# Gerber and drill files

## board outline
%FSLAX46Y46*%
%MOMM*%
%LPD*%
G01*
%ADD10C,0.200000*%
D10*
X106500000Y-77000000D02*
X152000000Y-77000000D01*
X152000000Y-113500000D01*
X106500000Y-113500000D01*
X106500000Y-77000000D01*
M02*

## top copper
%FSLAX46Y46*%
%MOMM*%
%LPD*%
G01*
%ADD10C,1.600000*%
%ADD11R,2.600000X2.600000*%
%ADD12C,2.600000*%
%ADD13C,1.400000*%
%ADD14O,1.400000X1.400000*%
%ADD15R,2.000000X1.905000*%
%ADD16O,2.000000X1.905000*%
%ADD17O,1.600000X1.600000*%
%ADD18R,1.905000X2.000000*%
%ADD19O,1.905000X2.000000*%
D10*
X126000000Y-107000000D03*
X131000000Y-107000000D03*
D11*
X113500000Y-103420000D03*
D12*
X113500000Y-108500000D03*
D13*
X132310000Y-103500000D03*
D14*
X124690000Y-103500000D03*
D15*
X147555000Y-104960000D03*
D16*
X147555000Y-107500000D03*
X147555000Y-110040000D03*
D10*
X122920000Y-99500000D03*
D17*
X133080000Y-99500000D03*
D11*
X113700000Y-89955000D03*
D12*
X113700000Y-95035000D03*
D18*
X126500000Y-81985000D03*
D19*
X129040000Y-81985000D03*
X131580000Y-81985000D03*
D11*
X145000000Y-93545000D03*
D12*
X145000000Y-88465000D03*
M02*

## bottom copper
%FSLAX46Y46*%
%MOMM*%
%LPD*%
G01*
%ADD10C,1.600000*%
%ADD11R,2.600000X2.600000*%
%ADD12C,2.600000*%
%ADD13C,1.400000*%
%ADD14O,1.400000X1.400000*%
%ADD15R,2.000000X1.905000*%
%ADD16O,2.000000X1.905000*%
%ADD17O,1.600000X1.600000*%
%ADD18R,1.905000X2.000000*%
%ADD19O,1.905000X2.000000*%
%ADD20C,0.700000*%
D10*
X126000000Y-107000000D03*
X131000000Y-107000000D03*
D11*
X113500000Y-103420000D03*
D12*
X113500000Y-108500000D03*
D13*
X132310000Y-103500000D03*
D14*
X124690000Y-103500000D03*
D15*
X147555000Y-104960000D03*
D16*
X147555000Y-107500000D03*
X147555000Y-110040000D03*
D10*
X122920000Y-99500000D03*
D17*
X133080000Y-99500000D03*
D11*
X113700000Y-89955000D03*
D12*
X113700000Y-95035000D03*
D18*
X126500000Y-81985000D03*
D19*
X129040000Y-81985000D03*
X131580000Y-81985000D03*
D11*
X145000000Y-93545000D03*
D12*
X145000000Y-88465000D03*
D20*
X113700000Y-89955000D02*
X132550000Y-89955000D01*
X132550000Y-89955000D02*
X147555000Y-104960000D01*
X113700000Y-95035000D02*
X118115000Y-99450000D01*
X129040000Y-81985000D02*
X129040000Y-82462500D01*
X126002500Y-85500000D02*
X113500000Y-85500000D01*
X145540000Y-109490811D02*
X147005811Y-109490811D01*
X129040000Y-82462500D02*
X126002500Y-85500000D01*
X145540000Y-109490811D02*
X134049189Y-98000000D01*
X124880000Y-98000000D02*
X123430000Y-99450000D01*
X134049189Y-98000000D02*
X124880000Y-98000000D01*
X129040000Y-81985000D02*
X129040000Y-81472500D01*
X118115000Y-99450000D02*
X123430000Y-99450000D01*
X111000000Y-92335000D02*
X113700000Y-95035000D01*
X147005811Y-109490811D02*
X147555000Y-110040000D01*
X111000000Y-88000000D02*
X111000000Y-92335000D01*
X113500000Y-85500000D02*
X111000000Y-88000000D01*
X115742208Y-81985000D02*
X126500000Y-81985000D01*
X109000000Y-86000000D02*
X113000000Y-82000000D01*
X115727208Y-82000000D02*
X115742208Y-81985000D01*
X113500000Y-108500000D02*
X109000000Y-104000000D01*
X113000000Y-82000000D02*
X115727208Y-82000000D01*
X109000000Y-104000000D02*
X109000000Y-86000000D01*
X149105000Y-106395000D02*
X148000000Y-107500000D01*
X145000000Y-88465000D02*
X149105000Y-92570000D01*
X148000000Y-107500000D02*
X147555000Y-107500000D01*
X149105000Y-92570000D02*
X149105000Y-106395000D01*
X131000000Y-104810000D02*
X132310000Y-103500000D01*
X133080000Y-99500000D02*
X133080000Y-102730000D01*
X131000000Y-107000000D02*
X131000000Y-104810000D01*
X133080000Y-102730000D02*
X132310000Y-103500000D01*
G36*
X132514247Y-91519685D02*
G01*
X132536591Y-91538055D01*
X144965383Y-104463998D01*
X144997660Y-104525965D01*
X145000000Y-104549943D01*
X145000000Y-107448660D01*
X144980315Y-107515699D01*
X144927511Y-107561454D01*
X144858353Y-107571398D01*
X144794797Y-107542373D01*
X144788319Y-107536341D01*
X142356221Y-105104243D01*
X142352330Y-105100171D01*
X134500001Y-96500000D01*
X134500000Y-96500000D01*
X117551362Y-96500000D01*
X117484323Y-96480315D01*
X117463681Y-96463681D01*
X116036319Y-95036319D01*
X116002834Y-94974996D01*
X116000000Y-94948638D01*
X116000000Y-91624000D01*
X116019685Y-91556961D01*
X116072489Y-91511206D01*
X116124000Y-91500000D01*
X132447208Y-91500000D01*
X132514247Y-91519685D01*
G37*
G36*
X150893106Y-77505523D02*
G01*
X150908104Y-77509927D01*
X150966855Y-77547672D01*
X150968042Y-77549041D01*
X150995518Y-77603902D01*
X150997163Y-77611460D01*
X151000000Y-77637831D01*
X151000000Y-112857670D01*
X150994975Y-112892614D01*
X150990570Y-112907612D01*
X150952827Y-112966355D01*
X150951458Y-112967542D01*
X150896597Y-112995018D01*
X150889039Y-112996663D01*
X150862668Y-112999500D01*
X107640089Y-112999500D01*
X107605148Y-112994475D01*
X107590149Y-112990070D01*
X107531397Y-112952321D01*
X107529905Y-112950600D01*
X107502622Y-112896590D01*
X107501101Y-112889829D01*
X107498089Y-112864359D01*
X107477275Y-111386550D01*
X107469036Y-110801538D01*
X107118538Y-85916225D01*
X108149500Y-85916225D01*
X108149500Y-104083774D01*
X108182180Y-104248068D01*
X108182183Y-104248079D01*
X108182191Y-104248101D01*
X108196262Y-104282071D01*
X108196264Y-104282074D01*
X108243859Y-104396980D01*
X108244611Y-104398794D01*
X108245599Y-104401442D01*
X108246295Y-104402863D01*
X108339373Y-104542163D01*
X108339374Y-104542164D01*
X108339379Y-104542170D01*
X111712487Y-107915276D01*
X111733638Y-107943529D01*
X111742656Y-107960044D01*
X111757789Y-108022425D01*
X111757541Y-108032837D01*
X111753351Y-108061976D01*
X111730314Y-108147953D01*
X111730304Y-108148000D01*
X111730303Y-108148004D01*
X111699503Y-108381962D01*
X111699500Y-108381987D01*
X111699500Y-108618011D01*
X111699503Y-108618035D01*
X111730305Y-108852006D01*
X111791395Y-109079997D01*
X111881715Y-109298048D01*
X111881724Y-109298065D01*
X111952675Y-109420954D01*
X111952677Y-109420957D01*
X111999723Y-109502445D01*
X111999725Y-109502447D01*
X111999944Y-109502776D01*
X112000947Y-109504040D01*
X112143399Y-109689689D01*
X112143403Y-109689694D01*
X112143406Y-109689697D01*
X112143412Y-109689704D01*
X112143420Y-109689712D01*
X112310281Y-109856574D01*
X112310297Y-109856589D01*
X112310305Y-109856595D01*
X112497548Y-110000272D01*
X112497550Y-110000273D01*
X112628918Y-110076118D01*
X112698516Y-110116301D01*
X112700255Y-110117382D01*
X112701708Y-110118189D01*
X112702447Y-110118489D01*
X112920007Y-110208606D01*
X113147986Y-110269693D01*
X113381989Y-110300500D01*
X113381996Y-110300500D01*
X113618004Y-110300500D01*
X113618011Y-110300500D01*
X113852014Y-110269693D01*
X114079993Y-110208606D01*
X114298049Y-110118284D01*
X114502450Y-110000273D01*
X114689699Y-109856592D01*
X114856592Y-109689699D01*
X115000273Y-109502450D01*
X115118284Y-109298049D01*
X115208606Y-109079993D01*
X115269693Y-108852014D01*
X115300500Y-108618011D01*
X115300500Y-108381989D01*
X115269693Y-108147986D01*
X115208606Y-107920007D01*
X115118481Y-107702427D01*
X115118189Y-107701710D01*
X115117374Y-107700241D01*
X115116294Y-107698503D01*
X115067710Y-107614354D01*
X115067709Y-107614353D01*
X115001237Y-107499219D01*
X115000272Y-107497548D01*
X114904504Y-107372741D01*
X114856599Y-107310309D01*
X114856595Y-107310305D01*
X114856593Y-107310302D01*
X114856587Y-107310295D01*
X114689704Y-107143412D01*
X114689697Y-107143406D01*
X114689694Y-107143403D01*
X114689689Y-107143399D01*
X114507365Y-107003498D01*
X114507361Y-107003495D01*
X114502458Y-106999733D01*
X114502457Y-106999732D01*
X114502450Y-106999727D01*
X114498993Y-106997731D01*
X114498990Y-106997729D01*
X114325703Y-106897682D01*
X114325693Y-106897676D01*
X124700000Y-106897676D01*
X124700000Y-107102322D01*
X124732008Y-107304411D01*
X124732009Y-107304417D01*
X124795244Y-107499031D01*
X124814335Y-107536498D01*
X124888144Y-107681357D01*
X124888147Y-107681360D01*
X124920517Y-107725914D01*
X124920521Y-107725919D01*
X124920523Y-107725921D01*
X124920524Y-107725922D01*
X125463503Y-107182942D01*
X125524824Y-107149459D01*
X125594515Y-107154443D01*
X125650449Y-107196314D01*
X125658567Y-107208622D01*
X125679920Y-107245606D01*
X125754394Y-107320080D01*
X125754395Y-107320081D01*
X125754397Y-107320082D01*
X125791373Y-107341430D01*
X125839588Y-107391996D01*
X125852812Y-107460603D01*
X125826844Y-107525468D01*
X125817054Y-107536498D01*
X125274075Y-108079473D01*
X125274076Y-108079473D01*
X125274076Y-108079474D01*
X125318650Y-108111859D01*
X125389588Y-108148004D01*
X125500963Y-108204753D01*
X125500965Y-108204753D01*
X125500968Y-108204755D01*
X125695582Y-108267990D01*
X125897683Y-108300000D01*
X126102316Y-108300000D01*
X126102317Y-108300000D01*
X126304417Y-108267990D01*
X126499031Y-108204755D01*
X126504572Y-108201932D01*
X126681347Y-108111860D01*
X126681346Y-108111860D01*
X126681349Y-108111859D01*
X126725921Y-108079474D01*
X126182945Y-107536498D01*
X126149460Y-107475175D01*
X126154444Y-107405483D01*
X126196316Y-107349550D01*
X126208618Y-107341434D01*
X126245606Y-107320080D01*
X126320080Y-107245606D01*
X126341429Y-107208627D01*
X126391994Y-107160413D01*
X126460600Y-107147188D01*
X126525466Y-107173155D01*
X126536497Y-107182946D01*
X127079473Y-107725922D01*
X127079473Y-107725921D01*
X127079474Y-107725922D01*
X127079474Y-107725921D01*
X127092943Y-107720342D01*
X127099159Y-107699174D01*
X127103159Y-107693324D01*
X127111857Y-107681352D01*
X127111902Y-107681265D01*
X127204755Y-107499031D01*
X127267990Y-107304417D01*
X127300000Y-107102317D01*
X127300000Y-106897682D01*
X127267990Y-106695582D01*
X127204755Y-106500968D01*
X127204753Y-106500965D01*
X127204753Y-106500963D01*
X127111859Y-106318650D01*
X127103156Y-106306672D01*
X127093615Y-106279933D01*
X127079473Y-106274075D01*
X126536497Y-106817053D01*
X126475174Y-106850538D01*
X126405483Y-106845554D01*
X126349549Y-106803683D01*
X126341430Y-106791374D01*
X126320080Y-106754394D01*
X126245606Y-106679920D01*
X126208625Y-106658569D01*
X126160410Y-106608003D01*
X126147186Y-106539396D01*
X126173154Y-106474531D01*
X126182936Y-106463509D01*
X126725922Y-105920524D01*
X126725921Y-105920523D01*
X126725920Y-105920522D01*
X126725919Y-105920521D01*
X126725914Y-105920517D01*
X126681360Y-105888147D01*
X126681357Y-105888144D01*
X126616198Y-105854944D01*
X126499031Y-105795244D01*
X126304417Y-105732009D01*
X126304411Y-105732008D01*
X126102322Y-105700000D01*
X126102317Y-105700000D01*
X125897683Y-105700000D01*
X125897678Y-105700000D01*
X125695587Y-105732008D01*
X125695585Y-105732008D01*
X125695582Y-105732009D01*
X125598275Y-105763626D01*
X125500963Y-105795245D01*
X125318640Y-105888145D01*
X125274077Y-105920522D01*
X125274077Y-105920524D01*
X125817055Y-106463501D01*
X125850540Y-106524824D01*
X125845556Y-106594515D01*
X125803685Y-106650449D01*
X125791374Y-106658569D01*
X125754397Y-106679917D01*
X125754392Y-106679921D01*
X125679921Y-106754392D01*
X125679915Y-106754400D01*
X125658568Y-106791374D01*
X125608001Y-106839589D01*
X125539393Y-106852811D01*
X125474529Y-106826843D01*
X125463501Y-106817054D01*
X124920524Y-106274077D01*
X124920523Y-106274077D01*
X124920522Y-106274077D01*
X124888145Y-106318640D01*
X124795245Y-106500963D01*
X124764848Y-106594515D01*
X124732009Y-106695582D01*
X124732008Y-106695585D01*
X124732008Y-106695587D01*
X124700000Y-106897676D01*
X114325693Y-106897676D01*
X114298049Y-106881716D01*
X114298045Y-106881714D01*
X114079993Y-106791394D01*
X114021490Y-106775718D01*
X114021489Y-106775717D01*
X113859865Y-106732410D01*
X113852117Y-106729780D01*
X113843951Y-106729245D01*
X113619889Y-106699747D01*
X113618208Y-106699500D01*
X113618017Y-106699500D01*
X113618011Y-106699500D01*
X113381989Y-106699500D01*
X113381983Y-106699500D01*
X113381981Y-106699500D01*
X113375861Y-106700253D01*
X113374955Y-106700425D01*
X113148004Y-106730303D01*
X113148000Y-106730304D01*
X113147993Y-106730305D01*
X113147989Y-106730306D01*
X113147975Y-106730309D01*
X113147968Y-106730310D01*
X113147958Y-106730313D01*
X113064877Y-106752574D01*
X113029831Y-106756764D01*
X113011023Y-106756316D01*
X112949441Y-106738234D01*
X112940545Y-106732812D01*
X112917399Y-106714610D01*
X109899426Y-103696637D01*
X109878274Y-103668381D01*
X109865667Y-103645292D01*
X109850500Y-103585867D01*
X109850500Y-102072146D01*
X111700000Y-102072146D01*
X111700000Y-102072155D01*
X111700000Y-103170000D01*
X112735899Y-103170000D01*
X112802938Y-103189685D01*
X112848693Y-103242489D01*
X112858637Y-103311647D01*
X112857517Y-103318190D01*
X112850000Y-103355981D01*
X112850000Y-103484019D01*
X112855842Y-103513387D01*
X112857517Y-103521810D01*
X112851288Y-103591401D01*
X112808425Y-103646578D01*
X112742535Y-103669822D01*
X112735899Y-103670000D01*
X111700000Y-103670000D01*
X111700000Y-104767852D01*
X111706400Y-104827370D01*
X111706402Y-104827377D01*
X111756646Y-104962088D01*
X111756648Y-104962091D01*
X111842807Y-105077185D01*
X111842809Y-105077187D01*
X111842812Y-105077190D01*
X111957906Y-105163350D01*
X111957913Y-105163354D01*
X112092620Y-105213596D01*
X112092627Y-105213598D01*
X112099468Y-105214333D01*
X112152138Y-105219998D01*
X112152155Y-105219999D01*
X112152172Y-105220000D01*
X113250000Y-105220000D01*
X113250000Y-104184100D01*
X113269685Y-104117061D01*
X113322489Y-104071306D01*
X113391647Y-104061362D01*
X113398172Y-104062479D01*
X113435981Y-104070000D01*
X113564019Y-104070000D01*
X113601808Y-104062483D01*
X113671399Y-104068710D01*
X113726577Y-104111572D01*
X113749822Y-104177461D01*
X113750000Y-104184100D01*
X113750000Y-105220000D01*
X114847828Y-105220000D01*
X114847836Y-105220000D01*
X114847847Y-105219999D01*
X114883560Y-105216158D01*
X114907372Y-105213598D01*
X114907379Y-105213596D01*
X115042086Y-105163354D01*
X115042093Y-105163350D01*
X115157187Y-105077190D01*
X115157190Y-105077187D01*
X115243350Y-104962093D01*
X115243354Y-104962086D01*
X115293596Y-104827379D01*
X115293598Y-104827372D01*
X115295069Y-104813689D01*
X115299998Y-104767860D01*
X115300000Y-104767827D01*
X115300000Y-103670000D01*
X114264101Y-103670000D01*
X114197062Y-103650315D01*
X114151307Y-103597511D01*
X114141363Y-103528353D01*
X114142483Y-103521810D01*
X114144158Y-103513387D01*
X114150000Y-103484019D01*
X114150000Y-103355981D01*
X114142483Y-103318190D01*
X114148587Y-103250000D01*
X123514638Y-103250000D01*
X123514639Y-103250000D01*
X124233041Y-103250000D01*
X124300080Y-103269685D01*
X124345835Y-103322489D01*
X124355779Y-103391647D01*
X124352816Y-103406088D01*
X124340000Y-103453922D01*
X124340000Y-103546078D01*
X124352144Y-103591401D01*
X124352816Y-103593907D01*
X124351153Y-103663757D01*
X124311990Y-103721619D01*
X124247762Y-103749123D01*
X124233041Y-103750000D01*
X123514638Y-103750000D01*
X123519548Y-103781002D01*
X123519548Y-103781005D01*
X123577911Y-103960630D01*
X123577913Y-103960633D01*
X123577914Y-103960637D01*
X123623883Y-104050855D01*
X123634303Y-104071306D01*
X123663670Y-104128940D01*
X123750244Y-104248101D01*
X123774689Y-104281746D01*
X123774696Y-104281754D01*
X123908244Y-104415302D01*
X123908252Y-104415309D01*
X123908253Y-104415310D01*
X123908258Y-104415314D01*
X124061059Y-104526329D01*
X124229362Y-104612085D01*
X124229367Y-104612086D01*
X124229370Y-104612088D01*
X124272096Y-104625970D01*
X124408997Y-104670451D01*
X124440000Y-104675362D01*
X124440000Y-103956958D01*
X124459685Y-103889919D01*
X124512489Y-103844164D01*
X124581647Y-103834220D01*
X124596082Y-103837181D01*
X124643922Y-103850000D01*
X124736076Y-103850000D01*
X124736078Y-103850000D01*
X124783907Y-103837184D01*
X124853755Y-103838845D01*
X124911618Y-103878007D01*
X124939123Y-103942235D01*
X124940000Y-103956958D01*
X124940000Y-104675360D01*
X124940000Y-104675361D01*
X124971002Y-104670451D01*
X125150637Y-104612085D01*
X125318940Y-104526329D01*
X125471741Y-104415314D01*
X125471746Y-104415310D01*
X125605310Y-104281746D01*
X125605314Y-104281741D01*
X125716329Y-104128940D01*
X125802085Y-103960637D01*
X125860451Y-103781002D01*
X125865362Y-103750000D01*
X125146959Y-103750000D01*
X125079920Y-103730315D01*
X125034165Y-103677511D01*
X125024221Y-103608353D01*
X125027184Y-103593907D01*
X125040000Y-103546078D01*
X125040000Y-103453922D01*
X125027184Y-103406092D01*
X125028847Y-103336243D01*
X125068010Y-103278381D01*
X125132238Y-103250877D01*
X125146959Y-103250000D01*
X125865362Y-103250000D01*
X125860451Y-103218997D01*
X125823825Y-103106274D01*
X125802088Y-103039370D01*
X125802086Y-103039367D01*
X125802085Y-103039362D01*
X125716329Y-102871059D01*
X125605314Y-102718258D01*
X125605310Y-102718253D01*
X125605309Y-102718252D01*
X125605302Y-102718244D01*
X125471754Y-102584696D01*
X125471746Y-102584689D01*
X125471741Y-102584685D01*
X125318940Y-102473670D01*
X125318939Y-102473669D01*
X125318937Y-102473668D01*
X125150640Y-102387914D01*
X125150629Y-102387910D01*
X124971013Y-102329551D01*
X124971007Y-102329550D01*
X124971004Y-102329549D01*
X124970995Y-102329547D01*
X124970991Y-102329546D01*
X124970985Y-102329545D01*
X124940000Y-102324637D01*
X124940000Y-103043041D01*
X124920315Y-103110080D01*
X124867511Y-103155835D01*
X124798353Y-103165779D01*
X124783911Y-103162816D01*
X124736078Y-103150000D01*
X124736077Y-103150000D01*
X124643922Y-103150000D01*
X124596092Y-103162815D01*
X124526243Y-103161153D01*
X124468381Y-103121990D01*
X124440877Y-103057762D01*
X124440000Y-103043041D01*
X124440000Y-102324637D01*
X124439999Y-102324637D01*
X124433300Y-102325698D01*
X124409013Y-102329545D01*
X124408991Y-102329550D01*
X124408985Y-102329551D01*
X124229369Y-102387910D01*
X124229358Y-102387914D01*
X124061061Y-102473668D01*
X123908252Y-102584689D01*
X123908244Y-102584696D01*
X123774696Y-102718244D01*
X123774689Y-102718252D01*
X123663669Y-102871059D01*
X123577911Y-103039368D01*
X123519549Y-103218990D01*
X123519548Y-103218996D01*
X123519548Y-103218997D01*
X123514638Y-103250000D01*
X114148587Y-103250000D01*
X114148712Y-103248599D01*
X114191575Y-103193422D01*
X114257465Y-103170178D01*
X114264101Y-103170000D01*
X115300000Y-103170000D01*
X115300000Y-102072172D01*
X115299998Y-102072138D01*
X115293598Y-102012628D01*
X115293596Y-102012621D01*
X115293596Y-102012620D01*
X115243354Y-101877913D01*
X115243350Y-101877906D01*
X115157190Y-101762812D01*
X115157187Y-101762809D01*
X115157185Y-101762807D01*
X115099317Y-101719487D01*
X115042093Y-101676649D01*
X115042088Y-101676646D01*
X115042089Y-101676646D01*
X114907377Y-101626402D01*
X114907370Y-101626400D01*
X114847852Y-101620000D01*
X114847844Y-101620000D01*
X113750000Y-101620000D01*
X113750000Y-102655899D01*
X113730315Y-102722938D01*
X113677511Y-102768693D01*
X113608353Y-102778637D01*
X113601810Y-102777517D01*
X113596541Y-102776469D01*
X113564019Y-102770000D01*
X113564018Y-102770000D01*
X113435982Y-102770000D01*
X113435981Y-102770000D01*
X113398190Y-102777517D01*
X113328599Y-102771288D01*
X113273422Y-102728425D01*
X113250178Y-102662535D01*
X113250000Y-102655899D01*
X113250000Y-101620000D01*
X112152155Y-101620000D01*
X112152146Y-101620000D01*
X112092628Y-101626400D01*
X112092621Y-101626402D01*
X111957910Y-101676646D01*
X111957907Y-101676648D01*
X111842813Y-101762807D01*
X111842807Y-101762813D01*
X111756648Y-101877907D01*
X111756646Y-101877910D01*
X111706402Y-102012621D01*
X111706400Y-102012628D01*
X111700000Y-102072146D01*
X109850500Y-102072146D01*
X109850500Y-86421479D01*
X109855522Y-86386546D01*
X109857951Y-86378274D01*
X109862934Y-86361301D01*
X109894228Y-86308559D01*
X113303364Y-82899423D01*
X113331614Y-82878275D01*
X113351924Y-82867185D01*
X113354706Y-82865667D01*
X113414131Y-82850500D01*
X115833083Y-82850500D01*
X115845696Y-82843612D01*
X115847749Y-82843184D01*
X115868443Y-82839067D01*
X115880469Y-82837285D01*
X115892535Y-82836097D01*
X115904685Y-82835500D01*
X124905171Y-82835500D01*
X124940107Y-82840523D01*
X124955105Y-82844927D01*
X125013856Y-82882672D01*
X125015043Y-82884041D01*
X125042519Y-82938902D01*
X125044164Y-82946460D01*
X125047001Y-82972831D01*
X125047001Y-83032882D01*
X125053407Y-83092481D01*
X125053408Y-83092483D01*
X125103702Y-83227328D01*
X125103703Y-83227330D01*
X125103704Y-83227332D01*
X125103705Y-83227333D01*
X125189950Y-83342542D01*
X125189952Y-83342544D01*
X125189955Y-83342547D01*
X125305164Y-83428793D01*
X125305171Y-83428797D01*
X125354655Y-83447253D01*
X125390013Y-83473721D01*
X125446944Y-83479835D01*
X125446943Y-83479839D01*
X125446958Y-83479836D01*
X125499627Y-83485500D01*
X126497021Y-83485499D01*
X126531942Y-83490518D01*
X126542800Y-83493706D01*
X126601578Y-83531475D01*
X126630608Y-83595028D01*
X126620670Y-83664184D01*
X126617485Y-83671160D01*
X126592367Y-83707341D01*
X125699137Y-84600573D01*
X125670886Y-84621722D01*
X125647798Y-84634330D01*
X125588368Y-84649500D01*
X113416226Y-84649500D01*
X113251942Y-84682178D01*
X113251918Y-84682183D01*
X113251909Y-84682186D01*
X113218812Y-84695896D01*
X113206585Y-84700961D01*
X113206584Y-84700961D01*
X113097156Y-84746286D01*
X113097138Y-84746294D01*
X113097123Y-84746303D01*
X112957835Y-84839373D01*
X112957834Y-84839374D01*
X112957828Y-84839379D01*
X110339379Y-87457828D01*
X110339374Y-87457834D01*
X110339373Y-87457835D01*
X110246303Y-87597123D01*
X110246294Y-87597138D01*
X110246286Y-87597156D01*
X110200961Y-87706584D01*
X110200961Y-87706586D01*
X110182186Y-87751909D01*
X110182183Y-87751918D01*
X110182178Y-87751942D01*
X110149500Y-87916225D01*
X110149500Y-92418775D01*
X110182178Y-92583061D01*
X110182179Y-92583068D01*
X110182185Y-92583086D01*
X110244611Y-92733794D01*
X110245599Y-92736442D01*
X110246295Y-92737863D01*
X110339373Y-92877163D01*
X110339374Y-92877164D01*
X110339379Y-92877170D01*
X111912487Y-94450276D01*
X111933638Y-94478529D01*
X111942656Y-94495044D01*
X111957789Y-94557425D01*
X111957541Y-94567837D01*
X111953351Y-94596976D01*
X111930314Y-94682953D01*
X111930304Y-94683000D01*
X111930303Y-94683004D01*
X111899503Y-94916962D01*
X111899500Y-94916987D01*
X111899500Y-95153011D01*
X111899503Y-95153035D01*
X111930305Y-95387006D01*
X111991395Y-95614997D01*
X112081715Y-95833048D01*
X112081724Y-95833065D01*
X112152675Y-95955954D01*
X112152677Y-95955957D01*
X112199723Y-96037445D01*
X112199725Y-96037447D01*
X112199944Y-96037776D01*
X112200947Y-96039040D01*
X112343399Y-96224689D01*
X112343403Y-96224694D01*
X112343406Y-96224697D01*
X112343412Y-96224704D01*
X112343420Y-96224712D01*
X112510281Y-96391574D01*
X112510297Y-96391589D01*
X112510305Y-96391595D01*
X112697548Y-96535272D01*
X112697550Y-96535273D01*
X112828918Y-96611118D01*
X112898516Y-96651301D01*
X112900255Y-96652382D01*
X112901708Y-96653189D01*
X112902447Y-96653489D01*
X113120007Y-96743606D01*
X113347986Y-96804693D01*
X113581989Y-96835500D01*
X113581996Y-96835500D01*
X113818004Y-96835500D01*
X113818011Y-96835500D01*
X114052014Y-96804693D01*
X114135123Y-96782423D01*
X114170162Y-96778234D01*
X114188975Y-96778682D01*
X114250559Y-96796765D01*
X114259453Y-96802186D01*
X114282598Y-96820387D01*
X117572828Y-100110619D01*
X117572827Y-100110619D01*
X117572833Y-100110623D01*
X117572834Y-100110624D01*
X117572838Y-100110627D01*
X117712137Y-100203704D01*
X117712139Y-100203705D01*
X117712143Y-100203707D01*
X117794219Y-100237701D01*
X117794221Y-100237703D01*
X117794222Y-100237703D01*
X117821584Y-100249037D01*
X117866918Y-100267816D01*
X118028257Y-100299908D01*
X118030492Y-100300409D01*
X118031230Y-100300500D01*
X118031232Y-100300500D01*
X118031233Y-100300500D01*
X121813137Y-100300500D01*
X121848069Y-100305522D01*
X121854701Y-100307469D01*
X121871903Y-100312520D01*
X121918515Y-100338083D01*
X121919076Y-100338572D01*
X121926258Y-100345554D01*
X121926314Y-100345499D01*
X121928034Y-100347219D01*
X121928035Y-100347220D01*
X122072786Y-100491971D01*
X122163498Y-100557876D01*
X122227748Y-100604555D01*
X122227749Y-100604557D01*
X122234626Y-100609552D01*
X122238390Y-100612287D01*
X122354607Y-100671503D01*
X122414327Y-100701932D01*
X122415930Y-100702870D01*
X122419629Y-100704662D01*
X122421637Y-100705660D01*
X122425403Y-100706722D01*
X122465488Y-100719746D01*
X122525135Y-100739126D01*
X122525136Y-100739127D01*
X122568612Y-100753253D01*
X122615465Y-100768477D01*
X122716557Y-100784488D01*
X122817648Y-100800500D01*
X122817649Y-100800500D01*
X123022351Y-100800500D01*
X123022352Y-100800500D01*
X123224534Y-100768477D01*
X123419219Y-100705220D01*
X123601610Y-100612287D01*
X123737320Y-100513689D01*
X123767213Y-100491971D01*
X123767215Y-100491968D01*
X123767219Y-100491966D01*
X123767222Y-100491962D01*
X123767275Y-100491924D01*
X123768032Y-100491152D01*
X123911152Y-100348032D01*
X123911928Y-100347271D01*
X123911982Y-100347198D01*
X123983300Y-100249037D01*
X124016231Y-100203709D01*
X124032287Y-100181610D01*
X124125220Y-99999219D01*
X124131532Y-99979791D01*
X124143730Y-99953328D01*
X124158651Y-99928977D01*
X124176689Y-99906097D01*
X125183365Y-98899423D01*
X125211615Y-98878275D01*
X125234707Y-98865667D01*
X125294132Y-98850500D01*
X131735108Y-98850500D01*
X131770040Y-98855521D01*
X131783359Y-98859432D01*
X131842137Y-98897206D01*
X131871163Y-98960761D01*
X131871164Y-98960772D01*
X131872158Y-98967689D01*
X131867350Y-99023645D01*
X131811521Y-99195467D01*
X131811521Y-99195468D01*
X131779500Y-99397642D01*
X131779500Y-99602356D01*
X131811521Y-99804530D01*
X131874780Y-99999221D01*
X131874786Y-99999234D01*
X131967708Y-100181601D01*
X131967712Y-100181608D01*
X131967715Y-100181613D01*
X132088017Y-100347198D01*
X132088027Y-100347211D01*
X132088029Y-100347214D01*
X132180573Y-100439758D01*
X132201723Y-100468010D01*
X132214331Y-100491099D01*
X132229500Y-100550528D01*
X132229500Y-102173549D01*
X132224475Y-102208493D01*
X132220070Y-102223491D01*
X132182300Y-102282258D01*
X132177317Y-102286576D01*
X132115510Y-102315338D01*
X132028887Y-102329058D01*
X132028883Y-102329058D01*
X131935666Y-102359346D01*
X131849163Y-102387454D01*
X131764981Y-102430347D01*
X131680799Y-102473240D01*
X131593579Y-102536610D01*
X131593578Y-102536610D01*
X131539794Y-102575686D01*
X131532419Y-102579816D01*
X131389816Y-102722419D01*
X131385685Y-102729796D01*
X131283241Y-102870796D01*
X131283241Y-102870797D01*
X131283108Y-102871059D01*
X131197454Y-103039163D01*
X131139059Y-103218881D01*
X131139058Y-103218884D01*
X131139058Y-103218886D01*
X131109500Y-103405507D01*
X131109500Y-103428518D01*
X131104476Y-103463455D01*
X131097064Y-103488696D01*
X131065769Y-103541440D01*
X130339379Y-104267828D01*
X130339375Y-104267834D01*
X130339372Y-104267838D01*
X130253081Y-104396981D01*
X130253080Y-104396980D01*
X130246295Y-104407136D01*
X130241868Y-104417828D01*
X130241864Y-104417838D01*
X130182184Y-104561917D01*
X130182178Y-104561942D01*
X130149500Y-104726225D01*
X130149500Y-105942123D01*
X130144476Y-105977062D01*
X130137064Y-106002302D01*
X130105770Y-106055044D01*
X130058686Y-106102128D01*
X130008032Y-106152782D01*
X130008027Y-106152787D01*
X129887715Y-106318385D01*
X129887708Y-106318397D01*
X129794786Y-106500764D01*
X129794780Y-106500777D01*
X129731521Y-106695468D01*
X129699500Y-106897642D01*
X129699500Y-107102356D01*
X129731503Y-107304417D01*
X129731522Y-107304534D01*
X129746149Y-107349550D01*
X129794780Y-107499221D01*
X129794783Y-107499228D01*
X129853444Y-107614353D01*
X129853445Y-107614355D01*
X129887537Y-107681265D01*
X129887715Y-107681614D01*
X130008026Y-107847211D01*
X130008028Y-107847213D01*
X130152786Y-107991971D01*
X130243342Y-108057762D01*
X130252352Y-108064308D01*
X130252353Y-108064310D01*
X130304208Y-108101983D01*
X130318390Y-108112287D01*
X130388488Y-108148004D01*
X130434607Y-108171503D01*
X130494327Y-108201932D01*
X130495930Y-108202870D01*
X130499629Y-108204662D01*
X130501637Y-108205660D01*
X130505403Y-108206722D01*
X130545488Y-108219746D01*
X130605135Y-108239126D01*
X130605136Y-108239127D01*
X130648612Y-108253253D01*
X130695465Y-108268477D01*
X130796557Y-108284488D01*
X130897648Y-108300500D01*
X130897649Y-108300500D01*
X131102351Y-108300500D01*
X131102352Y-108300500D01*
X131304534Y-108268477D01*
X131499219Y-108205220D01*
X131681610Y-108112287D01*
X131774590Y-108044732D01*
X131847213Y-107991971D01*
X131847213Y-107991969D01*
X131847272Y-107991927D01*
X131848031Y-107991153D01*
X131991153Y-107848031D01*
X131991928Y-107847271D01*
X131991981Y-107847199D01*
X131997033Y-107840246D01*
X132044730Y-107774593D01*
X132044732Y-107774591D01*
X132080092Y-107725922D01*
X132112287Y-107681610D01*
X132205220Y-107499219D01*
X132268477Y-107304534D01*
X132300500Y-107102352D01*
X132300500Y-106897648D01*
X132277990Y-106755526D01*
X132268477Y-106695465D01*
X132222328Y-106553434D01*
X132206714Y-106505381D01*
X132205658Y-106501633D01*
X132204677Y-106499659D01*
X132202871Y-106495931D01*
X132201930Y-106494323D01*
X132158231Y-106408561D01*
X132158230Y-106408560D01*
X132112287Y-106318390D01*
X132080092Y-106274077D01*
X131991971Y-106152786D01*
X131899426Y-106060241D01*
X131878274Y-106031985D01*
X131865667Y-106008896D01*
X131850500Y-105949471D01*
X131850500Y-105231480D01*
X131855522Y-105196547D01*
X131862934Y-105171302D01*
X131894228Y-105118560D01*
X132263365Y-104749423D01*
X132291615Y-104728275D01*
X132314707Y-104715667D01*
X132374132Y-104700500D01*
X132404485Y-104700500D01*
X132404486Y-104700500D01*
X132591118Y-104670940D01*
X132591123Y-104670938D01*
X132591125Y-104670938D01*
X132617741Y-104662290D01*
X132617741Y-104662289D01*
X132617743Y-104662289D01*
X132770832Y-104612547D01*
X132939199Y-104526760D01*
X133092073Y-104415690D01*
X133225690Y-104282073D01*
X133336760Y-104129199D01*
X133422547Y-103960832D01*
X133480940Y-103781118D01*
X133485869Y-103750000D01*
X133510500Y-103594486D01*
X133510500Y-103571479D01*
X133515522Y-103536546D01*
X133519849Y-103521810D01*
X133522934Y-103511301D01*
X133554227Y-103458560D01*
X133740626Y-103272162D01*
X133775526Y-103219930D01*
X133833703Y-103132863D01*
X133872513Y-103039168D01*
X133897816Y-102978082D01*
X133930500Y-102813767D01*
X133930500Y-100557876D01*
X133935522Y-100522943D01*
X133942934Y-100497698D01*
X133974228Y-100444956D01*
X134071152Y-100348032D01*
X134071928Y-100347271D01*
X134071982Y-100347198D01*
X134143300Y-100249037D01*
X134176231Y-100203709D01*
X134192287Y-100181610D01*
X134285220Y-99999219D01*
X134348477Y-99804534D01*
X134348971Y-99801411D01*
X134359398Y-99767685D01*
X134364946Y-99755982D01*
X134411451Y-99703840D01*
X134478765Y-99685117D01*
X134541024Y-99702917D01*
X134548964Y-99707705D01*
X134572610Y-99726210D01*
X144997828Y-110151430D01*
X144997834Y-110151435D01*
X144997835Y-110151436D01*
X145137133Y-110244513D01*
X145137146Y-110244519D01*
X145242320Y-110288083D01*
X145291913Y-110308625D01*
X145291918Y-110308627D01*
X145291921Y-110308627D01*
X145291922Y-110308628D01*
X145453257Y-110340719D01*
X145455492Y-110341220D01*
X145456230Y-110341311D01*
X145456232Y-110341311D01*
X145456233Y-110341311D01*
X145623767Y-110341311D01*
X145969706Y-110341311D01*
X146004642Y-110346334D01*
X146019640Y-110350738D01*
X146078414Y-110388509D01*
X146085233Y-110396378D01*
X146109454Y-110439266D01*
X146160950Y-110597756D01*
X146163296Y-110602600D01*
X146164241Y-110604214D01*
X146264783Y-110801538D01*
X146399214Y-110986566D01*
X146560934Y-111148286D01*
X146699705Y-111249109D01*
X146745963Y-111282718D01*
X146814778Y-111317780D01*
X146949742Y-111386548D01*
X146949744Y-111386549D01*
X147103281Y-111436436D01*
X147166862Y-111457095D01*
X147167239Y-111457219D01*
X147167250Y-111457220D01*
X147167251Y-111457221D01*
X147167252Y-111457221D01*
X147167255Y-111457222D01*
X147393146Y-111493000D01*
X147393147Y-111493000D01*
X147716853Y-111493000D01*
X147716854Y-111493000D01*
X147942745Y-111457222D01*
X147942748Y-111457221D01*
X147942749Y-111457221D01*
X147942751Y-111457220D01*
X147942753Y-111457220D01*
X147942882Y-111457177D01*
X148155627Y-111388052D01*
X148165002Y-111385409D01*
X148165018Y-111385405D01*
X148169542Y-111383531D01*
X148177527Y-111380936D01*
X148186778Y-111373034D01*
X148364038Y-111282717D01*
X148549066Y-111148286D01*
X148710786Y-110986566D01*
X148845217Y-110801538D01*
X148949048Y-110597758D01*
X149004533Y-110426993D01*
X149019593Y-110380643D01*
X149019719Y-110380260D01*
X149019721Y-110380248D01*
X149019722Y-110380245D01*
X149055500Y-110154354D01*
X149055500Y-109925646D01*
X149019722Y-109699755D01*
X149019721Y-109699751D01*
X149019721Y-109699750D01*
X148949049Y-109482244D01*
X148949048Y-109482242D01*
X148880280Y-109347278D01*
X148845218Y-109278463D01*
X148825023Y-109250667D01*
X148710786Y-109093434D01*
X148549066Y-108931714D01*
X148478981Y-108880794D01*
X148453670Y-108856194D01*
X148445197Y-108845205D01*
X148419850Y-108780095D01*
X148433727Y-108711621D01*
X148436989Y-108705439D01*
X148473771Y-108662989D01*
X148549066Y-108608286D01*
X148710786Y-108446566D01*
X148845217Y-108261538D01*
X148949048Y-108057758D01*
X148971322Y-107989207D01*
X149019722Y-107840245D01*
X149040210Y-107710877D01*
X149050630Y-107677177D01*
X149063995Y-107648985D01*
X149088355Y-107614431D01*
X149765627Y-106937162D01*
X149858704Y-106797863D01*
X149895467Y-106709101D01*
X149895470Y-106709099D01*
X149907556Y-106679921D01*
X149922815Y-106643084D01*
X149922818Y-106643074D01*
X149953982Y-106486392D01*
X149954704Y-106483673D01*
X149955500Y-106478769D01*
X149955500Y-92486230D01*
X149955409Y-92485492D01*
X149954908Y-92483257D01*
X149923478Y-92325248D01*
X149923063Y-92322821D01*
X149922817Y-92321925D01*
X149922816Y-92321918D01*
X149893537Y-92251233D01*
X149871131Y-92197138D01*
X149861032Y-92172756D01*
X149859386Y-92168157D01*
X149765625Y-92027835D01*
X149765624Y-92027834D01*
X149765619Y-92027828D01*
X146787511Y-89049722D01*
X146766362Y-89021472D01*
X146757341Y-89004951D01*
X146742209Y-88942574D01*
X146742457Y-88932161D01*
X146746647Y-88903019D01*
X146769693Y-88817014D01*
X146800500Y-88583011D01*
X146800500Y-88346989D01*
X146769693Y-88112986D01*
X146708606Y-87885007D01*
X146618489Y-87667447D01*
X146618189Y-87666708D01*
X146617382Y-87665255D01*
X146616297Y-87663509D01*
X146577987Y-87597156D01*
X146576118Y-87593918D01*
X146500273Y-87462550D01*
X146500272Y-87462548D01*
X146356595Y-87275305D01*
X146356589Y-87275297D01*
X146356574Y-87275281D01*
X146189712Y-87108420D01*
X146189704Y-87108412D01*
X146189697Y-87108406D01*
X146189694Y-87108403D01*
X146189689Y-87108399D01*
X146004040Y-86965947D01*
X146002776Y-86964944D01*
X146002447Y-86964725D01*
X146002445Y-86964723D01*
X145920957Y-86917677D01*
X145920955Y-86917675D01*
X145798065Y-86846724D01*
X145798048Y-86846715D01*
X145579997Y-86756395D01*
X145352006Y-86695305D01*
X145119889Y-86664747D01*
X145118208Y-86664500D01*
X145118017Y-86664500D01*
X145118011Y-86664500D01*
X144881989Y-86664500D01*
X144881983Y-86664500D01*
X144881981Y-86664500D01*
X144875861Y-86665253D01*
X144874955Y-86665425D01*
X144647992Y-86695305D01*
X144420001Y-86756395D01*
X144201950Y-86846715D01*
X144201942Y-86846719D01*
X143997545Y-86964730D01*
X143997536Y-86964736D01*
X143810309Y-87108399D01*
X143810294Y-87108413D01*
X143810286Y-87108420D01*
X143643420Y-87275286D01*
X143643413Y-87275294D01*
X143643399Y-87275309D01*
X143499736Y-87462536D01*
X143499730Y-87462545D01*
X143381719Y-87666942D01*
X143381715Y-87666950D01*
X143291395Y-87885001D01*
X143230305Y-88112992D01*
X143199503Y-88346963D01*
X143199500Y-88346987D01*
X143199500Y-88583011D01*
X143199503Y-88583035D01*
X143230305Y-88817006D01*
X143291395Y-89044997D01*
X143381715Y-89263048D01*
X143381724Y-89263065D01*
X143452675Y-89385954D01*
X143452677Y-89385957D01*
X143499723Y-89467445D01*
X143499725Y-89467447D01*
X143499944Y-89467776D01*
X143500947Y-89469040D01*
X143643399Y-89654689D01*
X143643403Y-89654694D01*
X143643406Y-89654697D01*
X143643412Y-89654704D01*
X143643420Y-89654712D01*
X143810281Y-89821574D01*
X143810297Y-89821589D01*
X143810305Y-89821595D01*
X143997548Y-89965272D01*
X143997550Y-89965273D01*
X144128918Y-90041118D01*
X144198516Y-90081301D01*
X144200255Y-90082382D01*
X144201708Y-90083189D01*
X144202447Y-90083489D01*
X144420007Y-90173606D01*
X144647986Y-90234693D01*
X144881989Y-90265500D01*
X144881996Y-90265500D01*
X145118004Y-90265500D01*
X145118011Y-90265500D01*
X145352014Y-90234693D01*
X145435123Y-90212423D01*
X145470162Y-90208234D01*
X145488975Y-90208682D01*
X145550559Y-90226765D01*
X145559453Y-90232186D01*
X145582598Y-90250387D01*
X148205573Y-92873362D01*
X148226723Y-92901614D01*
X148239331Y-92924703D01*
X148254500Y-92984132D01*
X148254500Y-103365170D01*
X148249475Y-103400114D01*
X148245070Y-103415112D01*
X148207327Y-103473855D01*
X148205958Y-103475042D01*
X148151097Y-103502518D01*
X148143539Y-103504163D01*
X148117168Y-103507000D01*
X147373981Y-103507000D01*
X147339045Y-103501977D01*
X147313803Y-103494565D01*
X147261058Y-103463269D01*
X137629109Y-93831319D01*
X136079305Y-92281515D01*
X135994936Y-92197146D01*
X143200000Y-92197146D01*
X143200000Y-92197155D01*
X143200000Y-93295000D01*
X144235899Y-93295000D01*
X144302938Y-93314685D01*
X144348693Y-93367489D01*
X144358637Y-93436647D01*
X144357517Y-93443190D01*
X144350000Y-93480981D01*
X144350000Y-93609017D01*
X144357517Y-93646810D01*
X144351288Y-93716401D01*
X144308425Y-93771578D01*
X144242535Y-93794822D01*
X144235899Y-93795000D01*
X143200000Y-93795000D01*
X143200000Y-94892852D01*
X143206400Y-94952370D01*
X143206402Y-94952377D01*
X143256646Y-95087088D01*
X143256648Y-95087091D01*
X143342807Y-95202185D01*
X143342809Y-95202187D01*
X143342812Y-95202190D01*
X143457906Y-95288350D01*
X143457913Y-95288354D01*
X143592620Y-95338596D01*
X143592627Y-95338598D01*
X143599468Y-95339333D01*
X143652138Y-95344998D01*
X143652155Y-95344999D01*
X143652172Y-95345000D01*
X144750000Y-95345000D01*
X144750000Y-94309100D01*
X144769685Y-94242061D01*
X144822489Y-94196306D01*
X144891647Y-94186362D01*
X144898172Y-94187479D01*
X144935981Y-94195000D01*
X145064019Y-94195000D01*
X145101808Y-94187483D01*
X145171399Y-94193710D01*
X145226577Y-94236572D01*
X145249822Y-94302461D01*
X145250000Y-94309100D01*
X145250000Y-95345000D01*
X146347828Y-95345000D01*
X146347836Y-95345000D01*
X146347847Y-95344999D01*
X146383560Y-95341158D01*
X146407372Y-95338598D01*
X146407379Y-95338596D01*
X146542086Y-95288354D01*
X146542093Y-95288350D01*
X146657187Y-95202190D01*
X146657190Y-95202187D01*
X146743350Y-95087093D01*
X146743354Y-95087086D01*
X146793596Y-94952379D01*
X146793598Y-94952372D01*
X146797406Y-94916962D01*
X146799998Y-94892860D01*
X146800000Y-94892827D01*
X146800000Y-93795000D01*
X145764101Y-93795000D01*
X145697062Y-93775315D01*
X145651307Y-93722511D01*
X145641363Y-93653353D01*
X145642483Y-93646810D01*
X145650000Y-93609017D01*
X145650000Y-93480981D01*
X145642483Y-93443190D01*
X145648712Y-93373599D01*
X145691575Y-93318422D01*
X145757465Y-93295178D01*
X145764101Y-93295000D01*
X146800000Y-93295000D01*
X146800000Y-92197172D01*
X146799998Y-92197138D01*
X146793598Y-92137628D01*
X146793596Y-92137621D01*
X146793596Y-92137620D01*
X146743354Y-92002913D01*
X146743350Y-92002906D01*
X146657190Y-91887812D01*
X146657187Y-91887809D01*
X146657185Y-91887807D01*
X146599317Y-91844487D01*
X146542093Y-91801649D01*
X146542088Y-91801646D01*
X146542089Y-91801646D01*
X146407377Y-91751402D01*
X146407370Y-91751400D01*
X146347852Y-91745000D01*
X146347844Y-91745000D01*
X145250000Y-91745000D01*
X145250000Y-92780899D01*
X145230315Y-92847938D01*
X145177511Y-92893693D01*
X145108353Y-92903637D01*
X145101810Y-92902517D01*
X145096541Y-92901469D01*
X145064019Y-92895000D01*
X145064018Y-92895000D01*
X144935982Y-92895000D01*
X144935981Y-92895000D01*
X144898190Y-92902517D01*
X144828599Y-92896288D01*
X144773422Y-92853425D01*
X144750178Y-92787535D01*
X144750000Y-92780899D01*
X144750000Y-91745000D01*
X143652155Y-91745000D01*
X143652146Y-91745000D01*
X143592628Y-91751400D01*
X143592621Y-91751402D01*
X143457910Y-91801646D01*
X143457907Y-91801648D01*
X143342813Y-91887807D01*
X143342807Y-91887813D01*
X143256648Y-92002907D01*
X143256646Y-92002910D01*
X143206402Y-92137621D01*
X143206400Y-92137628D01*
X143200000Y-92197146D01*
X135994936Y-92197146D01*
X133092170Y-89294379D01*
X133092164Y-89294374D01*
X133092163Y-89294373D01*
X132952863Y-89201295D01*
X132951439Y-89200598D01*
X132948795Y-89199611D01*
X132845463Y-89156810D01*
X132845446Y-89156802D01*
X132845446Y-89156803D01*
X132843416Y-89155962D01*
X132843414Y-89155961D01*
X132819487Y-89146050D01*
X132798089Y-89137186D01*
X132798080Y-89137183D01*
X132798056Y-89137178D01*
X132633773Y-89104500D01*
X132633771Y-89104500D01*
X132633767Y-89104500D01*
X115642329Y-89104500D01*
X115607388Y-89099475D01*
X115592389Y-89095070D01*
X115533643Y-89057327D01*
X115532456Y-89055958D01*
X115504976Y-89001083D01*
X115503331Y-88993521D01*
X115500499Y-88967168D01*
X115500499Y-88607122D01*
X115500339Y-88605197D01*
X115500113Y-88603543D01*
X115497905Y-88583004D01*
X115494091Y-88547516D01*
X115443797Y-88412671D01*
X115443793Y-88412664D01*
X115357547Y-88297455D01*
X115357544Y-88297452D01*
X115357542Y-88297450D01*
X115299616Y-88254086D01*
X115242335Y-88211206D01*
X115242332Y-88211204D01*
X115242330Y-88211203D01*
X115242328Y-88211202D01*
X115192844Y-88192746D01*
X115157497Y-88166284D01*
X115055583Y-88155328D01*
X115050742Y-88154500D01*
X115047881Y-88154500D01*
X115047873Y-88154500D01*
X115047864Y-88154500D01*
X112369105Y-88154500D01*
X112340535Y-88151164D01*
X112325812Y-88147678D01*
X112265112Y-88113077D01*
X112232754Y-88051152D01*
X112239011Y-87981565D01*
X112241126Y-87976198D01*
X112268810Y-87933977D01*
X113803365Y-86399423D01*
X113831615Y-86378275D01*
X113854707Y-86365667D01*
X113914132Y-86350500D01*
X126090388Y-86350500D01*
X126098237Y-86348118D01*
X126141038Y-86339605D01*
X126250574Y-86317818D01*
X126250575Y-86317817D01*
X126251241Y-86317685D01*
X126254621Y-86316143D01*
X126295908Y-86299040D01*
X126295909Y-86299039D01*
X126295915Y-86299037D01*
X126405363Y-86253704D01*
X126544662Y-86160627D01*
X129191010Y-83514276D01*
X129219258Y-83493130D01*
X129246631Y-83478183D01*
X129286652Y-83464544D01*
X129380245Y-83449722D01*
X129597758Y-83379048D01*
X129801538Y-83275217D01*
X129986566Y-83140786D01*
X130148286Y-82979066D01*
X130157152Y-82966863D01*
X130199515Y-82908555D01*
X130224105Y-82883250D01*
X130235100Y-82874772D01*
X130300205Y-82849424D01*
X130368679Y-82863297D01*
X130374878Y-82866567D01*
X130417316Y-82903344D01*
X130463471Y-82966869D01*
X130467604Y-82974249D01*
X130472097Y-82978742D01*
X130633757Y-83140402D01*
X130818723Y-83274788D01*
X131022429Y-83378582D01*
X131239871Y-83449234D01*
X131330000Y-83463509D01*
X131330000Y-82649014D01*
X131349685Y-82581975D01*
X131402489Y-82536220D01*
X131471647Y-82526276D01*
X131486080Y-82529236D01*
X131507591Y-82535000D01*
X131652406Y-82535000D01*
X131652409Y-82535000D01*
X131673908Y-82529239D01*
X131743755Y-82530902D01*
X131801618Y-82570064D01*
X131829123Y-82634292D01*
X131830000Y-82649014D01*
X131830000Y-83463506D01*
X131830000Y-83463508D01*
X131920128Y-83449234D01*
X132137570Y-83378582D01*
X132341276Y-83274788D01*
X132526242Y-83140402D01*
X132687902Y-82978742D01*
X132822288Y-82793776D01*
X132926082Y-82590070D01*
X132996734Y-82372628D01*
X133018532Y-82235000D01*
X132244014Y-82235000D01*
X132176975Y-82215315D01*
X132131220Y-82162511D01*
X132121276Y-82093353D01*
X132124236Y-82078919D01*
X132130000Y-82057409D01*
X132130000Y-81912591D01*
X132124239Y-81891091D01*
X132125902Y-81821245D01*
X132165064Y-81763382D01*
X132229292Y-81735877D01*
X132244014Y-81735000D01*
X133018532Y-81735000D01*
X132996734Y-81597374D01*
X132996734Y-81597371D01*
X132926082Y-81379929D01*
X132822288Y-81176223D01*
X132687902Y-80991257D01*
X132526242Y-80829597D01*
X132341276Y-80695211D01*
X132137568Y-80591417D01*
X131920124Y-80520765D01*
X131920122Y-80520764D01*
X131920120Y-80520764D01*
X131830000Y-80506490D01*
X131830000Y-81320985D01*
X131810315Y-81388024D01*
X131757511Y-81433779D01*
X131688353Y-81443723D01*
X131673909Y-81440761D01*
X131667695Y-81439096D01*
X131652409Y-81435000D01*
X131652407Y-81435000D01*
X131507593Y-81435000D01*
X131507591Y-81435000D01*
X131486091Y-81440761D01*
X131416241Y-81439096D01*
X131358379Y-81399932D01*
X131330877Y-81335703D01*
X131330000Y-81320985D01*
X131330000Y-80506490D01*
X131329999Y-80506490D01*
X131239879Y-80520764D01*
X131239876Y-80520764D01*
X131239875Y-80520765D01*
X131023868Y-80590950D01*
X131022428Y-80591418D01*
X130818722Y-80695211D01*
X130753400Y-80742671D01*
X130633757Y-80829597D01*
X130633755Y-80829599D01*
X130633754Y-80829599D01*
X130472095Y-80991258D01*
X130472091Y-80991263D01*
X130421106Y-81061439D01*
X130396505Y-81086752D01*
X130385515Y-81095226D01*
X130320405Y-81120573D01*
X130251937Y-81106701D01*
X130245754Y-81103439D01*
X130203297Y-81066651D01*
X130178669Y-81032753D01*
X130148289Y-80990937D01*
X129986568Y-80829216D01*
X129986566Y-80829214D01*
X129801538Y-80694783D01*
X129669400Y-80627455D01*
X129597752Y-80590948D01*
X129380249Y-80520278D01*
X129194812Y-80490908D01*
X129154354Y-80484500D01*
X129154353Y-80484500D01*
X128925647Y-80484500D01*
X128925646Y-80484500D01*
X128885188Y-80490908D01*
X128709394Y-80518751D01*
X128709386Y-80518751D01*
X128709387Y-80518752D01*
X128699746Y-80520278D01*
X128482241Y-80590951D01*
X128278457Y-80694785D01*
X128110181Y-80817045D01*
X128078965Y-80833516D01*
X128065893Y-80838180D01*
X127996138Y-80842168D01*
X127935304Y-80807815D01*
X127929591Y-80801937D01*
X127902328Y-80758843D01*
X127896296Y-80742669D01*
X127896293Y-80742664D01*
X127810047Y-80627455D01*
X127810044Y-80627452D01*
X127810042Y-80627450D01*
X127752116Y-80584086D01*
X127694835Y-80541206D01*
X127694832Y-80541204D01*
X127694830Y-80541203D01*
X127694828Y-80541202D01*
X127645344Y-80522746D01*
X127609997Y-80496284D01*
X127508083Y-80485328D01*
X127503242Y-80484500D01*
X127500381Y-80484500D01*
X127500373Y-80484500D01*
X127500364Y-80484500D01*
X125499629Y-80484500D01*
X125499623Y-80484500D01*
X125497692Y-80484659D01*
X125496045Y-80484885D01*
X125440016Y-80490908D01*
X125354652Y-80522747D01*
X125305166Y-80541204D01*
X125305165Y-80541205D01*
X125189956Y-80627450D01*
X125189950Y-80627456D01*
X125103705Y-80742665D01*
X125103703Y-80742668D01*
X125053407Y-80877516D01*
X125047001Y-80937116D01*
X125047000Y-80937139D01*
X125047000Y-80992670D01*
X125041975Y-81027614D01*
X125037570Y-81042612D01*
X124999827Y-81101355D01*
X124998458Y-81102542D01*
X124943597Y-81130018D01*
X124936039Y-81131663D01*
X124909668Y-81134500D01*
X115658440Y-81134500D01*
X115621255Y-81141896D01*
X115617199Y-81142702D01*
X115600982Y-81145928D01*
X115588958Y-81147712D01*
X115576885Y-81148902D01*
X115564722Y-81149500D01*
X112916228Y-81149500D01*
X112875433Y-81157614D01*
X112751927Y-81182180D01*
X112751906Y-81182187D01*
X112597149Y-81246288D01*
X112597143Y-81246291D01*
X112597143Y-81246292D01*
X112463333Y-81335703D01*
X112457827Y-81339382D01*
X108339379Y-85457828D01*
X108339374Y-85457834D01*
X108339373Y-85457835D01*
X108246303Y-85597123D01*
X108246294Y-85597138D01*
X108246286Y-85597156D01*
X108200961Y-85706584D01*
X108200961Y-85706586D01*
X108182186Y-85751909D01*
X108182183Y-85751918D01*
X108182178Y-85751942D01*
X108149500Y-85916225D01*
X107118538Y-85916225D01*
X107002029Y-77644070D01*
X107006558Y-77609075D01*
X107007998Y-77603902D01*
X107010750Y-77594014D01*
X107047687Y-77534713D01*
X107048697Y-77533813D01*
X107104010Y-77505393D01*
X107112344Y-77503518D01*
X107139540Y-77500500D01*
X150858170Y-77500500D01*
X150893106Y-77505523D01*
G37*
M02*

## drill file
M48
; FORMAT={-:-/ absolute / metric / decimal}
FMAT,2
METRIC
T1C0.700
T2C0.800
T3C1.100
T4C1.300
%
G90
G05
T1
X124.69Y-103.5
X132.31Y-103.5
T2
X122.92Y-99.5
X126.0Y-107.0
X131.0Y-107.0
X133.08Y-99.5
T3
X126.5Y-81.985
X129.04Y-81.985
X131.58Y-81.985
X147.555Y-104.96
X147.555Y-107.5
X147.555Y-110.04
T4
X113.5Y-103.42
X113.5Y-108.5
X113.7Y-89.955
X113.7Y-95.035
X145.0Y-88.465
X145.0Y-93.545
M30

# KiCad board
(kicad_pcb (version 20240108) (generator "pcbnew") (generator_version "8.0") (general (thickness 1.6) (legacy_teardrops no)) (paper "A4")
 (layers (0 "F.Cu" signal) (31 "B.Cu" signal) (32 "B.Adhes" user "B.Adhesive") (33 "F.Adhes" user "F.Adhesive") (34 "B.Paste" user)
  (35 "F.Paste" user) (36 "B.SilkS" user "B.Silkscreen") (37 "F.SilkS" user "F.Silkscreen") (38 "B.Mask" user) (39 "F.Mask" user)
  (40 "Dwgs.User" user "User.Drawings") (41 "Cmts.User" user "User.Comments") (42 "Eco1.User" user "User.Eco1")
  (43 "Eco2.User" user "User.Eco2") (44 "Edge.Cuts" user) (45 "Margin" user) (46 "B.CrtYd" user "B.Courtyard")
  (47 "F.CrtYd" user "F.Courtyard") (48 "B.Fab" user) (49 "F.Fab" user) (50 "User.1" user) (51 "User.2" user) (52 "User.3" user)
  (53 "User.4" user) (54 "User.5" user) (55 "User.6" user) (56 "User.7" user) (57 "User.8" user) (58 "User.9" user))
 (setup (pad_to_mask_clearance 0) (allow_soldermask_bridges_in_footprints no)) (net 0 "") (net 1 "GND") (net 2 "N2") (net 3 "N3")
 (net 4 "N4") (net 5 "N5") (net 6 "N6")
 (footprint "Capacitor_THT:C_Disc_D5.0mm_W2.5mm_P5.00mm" (layer "F.Cu") (at 126 107)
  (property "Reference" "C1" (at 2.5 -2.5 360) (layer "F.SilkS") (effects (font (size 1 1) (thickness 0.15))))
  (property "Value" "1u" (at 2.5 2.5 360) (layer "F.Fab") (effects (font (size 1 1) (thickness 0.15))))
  (pad "1" thru_hole circle (at 0 0) (size 1.6 1.6) (drill 0.8) (layers "*.Cu" "*.Mask") (remove_unused_layers no) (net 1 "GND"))
  (pad "2" thru_hole circle (at 5 0) (size 1.6 1.6) (drill 0.8) (layers "*.Cu" "*.Mask") (remove_unused_layers no) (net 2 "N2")))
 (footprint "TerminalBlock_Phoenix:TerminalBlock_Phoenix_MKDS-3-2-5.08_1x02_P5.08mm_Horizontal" (layer "F.Cu") (at 113.5 103.42 -90)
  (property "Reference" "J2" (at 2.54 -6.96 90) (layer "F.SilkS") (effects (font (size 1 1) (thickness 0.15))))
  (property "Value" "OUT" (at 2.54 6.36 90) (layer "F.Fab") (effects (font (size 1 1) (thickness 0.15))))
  (pad "1" thru_hole rect (at 0 0 270) (size 2.6 2.6) (drill 1.3) (layers "*.Cu" "*.Mask") (remove_unused_layers no) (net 1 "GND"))
  (pad "2" thru_hole circle (at 5.08 0 270) (size 2.6 2.6) (drill 1.3) (layers "*.Cu" "*.Mask") (remove_unused_layers no) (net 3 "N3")))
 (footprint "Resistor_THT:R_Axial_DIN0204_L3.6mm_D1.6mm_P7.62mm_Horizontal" (layer "F.Cu") (at 132.31 103.5 180)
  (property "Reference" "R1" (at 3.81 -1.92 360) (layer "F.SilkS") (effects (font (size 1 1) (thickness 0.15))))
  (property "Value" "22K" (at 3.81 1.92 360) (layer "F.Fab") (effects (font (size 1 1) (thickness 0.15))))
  (pad "1" thru_hole circle (at 0 0 180) (size 1.4 1.4) (drill 0.7) (layers "*.Cu" "*.Mask") (remove_unused_layers no) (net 2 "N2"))
  (pad "2" thru_hole oval (at 7.62 0 180) (size 1.4 1.4) (drill 0.7) (layers "*.Cu" "*.Mask") (remove_unused_layers no) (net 1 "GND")))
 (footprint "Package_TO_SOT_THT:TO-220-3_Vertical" (layer "F.Cu") (at 147.555 104.96 -90)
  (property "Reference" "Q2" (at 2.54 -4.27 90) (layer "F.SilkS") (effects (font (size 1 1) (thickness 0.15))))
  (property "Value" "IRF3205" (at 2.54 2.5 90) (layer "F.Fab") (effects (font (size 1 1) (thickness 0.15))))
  (pad "1" thru_hole rect (at 0 0 270) (size 1.905 2) (drill 1.1) (layers "*.Cu" "*.Mask") (remove_unused_layers no) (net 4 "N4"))
  (pad "2" thru_hole oval (at 2.54 0 270) (size 1.905 2) (drill 1.1) (layers "*.Cu" "*.Mask") (remove_unused_layers no) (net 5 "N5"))
  (pad "3" thru_hole oval (at 5.08 0 270) (size 1.905 2) (drill 1.1) (layers "*.Cu" "*.Mask") (remove_unused_layers no) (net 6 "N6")))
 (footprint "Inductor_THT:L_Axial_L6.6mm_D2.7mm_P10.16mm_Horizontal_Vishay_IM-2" (layer "F.Cu") (at 122.92 99.5)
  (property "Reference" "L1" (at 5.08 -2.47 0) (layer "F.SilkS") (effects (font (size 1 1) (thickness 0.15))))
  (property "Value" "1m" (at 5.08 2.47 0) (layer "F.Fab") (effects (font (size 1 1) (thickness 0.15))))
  (pad "1" thru_hole circle (at 0 0) (size 1.6 1.6) (drill 0.8) (layers "*.Cu" "*.Mask") (remove_unused_layers no) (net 6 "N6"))
  (pad "2" thru_hole oval (at 10.16 0) (size 1.6 1.6) (drill 0.8) (layers "*.Cu" "*.Mask") (remove_unused_layers no) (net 2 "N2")))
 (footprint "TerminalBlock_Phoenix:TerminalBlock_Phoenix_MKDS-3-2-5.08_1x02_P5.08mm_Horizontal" (layer "F.Cu") (at 113.7 89.955 -90)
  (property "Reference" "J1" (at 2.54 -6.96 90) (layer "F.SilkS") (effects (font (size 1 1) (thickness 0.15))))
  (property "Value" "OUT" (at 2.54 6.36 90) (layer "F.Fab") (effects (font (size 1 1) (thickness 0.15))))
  (pad "1" thru_hole rect (at 0 0 270) (size 2.6 2.6) (drill 1.3) (layers "*.Cu" "*.Mask") (remove_unused_layers no) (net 4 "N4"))
  (pad "2" thru_hole circle (at 5.08 0 270) (size 2.6 2.6) (drill 1.3) (layers "*.Cu" "*.Mask") (remove_unused_layers no) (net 6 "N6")))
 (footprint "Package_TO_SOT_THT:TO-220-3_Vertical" (layer "F.Cu") (at 126.5 81.985)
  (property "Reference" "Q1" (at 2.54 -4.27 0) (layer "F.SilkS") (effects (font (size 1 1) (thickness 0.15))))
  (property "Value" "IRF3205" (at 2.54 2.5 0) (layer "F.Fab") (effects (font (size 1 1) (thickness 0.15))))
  (pad "1" thru_hole rect (at 0 0) (size 1.905 2) (drill 1.1) (layers "*.Cu" "*.Mask") (remove_unused_layers no) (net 3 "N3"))
  (pad "2" thru_hole oval (at 2.54 0) (size 1.905 2) (drill 1.1) (layers "*.Cu" "*.Mask") (remove_unused_layers no) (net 6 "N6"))
  (pad "3" thru_hole oval (at 5.08 0) (size 1.905 2) (drill 1.1) (layers "*.Cu" "*.Mask") (remove_unused_layers no) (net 1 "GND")))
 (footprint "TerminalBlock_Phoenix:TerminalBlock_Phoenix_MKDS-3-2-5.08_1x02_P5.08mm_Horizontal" (layer "F.Cu") (at 145 93.545 90)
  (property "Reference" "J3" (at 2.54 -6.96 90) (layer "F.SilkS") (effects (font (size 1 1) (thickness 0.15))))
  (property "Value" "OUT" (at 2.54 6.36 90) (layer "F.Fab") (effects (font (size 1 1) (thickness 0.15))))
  (pad "1" thru_hole rect (at 0 0 90) (size 2.6 2.6) (drill 1.3) (layers "*.Cu" "*.Mask") (remove_unused_layers no) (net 1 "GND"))
  (pad "2" thru_hole circle (at 5.08 0 90) (size 2.6 2.6) (drill 1.3) (layers "*.Cu" "*.Mask") (remove_unused_layers no) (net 5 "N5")))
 (gr_rect (start 106.5 77) (end 152 113.5) (stroke (width 0.2) (type default)) (fill none) (layer "Edge.Cuts"))
 (segment (start 113.7 89.955) (end 132.55 89.955) (width 0.7) (layer "B.Cu") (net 4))
 (segment (start 132.55 89.955) (end 147.555 104.96) (width 0.7) (layer "B.Cu") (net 4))
 (segment (start 113.7 95.035) (end 118.115 99.45) (width 0.7) (layer "B.Cu") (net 6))
 (segment (start 129.04 81.985) (end 129.04 82.4625) (width 0.7) (layer "B.Cu") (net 6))
 (segment (start 126.0025 85.5) (end 113.5 85.5) (width 0.7) (layer "B.Cu") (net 6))
 (segment (start 145.54 109.490811) (end 147.005811 109.490811) (width 0.7) (layer "B.Cu") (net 6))
 (segment (start 129.04 82.4625) (end 126.0025 85.5) (width 0.7) (layer "B.Cu") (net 6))
 (segment (start 145.54 109.490811) (end 134.049189 98) (width 0.7) (layer "B.Cu") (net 6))
 (segment (start 124.88 98) (end 123.43 99.45) (width 0.7) (layer "B.Cu") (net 6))
 (segment (start 134.049189 98) (end 124.88 98) (width 0.7) (layer "B.Cu") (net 6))
 (segment (start 129.04 81.985) (end 129.04 81.4725) (width 0.7) (layer "B.Cu") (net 6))
 (segment (start 118.115 99.45) (end 123.43 99.45) (width 0.7) (layer "B.Cu") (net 6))
 (segment (start 111 92.335) (end 113.7 95.035) (width 0.7) (layer "B.Cu") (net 6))
 (segment (start 147.005811 109.490811) (end 147.555 110.04) (width 0.7) (layer "B.Cu") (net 6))
 (segment (start 111 88) (end 111 92.335) (width 0.7) (layer "B.Cu") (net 6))
 (segment (start 113.5 85.5) (end 111 88) (width 0.7) (layer "B.Cu") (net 6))
 (segment (start 115.742208 81.985) (end 126.5 81.985) (width 0.7) (layer "B.Cu") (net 3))
 (segment (start 109 86) (end 113 82) (width 0.7) (layer "B.Cu") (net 3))
 (segment (start 115.727208 82) (end 115.742208 81.985) (width 0.7) (layer "B.Cu") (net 3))
 (segment (start 113.5 108.5) (end 109 104) (width 0.7) (layer "B.Cu") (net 3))
 (segment (start 113 82) (end 115.727208 82) (width 0.7) (layer "B.Cu") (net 3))
 (segment (start 109 104) (end 109 86) (width 0.7) (layer "B.Cu") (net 3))
 (segment (start 149.105 106.395) (end 148 107.5) (width 0.7) (layer "B.Cu") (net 5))
 (segment (start 145 88.465) (end 149.105 92.57) (width 0.7) (layer "B.Cu") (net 5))
 (segment (start 148 107.5) (end 147.555 107.5) (width 0.7) (layer "B.Cu") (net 5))
 (segment (start 149.105 92.57) (end 149.105 106.395) (width 0.7) (layer "B.Cu") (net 5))
 (segment (start 131 104.81) (end 132.31 103.5) (width 0.7) (layer "B.Cu") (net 2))
 (segment (start 133.08 99.5) (end 133.08 102.73) (width 0.7) (layer "B.Cu") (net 2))
 (segment (start 131 107) (end 131 104.81) (width 0.7) (layer "B.Cu") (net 2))
 (segment (start 133.08 102.73) (end 132.31 103.5) (width 0.7) (layer "B.Cu") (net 2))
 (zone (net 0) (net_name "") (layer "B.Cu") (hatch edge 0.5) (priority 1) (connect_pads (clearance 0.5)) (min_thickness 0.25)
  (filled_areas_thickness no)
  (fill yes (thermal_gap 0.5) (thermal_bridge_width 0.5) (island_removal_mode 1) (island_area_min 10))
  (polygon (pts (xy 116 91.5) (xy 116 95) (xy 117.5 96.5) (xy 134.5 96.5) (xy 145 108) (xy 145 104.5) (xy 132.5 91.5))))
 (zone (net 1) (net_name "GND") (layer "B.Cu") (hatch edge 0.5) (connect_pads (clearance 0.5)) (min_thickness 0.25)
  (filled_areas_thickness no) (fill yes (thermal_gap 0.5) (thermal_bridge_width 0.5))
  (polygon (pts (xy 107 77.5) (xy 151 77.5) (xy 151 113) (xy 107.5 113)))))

